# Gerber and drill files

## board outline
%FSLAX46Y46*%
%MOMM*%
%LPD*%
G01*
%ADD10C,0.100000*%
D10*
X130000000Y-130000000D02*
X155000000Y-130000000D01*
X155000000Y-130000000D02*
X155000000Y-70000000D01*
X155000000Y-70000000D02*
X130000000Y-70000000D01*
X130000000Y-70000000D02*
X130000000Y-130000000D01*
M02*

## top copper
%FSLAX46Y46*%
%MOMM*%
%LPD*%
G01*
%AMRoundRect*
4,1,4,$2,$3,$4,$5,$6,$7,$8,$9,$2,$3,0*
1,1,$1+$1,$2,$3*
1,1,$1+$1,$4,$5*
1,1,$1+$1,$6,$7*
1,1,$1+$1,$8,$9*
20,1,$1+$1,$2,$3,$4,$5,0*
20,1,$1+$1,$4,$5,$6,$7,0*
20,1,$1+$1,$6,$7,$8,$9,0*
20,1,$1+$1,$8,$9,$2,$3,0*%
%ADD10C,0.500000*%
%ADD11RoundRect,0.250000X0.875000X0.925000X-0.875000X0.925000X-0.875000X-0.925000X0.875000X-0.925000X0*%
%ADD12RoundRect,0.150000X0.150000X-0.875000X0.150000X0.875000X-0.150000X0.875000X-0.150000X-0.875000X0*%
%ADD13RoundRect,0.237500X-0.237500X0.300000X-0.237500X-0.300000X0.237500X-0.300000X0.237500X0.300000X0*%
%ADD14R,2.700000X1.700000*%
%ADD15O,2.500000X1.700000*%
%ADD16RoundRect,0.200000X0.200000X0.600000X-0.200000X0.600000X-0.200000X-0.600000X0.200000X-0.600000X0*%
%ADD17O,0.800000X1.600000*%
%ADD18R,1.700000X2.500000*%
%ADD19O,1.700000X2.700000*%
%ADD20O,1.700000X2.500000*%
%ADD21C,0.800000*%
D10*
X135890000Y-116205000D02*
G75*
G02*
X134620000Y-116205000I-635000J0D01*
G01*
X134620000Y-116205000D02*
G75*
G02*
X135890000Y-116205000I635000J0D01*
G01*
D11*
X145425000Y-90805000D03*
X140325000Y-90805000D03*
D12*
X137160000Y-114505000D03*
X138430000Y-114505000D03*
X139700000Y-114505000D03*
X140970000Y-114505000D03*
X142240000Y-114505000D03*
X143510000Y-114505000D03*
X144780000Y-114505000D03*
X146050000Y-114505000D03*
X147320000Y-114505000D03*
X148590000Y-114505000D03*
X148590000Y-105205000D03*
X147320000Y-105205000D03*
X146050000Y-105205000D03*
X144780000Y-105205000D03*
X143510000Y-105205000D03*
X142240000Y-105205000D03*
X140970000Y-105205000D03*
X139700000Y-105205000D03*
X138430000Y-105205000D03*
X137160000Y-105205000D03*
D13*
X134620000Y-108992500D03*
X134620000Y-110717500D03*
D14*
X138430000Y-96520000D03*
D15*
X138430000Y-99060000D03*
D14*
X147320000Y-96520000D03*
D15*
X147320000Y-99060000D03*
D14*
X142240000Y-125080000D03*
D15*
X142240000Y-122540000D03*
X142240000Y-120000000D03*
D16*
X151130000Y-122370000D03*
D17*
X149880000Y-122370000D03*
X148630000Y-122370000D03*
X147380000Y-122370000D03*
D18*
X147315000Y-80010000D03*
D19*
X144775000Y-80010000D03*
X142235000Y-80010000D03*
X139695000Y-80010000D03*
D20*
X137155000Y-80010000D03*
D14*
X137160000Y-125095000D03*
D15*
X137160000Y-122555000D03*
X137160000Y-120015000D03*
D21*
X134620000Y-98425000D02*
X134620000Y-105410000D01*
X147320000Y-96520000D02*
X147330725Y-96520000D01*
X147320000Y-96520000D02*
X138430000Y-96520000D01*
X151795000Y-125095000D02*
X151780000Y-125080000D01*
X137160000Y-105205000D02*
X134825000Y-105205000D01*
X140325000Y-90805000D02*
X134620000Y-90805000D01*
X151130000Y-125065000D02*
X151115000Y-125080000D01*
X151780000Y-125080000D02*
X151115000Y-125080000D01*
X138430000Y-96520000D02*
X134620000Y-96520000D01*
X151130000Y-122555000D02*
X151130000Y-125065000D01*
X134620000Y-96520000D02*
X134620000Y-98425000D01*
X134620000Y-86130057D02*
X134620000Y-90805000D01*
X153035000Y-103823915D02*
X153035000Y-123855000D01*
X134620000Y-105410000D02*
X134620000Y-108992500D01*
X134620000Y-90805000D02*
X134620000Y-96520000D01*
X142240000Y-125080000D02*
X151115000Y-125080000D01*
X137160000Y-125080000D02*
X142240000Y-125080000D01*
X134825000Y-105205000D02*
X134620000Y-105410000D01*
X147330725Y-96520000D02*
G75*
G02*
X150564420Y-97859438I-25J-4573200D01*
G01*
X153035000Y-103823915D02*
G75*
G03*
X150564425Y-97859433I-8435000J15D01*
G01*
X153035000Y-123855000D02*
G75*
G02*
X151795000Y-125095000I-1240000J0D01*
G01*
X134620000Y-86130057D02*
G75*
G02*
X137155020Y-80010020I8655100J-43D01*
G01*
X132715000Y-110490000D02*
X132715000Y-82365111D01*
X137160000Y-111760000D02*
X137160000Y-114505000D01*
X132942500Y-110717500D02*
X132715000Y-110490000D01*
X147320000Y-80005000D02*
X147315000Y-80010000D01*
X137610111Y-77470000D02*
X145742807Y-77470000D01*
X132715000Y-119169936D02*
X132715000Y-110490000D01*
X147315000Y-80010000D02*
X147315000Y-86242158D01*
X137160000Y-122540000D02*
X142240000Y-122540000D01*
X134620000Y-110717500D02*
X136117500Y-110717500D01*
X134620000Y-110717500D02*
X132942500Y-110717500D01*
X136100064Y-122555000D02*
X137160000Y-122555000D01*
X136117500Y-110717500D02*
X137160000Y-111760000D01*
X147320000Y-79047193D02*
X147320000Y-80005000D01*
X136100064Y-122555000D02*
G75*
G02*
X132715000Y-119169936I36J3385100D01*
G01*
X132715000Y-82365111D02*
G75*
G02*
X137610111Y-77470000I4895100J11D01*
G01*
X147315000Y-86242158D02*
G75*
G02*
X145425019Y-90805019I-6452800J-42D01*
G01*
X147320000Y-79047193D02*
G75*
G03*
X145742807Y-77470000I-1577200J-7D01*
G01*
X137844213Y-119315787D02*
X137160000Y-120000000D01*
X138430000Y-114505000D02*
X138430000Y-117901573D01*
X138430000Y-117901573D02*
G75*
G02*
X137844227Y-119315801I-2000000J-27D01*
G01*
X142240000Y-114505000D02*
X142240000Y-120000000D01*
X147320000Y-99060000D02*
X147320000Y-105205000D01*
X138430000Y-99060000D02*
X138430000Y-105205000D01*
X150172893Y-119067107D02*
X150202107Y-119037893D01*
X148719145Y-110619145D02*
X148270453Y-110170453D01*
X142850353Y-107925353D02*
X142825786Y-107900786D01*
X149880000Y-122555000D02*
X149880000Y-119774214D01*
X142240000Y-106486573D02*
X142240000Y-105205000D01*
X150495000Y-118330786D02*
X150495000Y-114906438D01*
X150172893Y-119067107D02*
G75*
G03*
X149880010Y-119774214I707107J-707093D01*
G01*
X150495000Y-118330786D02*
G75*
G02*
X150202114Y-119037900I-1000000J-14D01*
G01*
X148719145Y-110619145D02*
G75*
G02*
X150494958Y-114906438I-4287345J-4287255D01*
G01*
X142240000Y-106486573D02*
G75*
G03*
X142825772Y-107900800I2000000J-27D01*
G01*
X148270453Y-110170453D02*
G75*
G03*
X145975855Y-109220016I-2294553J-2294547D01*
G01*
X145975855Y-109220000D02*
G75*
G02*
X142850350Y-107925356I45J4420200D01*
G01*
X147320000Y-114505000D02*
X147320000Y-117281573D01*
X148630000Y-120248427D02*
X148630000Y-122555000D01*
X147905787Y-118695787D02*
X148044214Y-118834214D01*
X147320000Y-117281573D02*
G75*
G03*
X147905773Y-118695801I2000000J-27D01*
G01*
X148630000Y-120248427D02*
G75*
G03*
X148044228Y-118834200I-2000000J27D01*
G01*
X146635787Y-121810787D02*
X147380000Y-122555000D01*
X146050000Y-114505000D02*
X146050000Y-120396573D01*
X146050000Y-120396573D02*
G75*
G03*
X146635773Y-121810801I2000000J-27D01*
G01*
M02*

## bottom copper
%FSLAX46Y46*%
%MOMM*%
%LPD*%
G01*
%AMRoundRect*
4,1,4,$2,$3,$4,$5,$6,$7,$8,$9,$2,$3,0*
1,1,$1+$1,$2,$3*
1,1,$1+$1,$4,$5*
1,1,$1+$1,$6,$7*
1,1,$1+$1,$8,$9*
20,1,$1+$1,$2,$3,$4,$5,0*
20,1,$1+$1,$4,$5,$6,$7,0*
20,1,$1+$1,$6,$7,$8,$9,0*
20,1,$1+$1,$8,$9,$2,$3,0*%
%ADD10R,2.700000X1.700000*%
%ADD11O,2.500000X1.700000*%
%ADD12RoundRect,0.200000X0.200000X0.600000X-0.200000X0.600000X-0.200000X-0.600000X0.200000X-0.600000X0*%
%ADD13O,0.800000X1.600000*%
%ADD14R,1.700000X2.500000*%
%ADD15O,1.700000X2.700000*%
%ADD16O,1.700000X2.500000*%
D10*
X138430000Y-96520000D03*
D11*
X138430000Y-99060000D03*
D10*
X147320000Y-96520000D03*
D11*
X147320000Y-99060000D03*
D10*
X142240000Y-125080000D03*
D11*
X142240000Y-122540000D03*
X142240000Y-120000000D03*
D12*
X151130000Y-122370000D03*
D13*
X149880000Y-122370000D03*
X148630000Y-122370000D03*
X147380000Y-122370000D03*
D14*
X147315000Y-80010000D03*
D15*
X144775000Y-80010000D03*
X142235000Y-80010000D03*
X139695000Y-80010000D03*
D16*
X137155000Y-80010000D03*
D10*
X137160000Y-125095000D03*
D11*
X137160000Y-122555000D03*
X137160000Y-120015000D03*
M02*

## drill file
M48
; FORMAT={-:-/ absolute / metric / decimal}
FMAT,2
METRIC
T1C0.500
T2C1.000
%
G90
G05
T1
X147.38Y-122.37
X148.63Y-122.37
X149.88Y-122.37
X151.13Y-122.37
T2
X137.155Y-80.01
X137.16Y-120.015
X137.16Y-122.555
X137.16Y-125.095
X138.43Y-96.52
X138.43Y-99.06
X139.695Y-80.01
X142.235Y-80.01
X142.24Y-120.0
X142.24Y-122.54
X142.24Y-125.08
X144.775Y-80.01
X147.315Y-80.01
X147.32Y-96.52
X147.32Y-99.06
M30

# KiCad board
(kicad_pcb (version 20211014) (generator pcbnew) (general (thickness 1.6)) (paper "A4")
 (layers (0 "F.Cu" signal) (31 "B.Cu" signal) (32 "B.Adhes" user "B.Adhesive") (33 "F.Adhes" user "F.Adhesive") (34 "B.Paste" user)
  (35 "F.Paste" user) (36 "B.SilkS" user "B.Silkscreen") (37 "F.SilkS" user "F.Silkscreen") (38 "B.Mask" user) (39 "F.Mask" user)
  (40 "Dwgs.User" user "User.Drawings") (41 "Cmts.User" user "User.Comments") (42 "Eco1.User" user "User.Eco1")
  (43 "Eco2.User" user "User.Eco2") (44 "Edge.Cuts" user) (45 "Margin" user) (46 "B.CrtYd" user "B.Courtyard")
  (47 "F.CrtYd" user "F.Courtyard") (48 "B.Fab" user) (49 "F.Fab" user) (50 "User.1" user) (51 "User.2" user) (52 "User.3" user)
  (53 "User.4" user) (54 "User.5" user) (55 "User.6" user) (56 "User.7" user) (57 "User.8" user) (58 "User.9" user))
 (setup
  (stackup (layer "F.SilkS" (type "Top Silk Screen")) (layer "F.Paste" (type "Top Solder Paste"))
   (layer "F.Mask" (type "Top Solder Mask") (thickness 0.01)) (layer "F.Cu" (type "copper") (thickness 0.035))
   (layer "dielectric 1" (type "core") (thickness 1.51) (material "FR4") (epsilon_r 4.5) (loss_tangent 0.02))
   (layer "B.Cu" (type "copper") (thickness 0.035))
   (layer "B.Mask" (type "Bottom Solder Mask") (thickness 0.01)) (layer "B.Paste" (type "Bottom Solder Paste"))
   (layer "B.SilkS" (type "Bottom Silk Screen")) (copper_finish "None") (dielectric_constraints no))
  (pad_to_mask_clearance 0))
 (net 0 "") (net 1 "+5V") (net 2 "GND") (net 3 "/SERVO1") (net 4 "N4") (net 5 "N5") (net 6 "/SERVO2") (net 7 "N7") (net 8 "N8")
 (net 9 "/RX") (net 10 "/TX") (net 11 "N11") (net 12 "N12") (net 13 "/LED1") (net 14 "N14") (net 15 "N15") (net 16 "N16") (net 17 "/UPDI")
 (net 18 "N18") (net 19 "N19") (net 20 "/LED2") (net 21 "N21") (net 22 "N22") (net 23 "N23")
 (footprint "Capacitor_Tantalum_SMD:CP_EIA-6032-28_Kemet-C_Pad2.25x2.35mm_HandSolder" (layer "F.Cu") (at 142.875 90.805 180)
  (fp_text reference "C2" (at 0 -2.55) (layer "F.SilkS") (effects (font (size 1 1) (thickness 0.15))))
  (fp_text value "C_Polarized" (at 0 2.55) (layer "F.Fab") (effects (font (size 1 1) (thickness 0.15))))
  (pad "1" smd roundrect locked (at -2.55 0 180) (size 2.25 2.35) (layers "F.Cu" "F.Paste" "F.Mask") (roundrect_rratio 0.111111)
   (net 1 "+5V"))
  (pad "2" smd roundrect locked (at 2.55 0 180) (size 2.25 2.35) (layers "F.Cu" "F.Paste" "F.Mask") (roundrect_rratio 0.111111)
   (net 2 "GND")))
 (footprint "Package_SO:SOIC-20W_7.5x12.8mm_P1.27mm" (layer "F.Cu") (at 142.875 109.855 90)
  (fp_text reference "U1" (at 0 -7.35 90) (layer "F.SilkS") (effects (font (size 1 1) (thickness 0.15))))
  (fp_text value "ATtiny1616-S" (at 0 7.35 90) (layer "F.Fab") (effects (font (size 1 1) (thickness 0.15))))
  (pad "1" smd roundrect locked (at -4.65 -5.715 90) (size 2.05 0.6) (layers "F.Cu" "F.Paste" "F.Mask") (roundrect_rratio 0.25)
   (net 1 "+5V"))
  (pad "2" smd roundrect locked (at -4.65 -4.445 90) (size 2.05 0.6) (layers "F.Cu" "F.Paste" "F.Mask") (roundrect_rratio 0.25)
   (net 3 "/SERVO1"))
  (pad "3" smd roundrect locked (at -4.65 -3.175 90) (size 2.05 0.6) (layers "F.Cu" "F.Paste" "F.Mask") (roundrect_rratio 0.25) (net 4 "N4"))
  (pad "4" smd roundrect locked (at -4.65 -1.905 90) (size 2.05 0.6) (layers "F.Cu" "F.Paste" "F.Mask") (roundrect_rratio 0.25) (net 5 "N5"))
  (pad "5" smd roundrect locked (at -4.65 -0.635 90) (size 2.05 0.6) (layers "F.Cu" "F.Paste" "F.Mask") (roundrect_rratio 0.25)
   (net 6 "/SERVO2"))
  (pad "6" smd roundrect locked (at -4.65 0.635 90) (size 2.05 0.6) (layers "F.Cu" "F.Paste" "F.Mask") (roundrect_rratio 0.25) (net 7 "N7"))
  (pad "7" smd roundrect locked (at -4.65 1.905 90) (size 2.05 0.6) (layers "F.Cu" "F.Paste" "F.Mask") (roundrect_rratio 0.25) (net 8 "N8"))
  (pad "8" smd roundrect locked (at -4.65 3.175 90) (size 2.05 0.6) (layers "F.Cu" "F.Paste" "F.Mask") (roundrect_rratio 0.25) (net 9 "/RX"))
  (pad "9" smd roundrect locked (at -4.65 4.445 90) (size 2.05 0.6) (layers "F.Cu" "F.Paste" "F.Mask") (roundrect_rratio 0.25)
   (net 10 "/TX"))
  (pad "10" smd roundrect locked (at -4.65 5.715 90) (size 2.05 0.6) (layers "F.Cu" "F.Paste" "F.Mask") (roundrect_rratio 0.25)
   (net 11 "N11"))
  (pad "11" smd roundrect locked (at 4.65 5.715 90) (size 2.05 0.6) (layers "F.Cu" "F.Paste" "F.Mask") (roundrect_rratio 0.25)
   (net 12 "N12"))
  (pad "12" smd roundrect locked (at 4.65 4.445 90) (size 2.05 0.6) (layers "F.Cu" "F.Paste" "F.Mask") (roundrect_rratio 0.25)
   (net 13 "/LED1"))
  (pad "13" smd roundrect locked (at 4.65 3.175 90) (size 2.05 0.6) (layers "F.Cu" "F.Paste" "F.Mask") (roundrect_rratio 0.25)
   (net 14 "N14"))
  (pad "14" smd roundrect locked (at 4.65 1.905 90) (size 2.05 0.6) (layers "F.Cu" "F.Paste" "F.Mask") (roundrect_rratio 0.25)
   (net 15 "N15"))
  (pad "15" smd roundrect locked (at 4.65 0.635 90) (size 2.05 0.6) (layers "F.Cu" "F.Paste" "F.Mask") (roundrect_rratio 0.25)
   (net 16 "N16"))
  (pad "16" smd roundrect locked (at 4.65 -0.635 90) (size 2.05 0.6) (layers "F.Cu" "F.Paste" "F.Mask") (roundrect_rratio 0.25)
   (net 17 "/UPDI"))
  (pad "17" smd roundrect locked (at 4.65 -1.905 90) (size 2.05 0.6) (layers "F.Cu" "F.Paste" "F.Mask") (roundrect_rratio 0.25)
   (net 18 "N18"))
  (pad "18" smd roundrect locked (at 4.65 -3.175 90) (size 2.05 0.6) (layers "F.Cu" "F.Paste" "F.Mask") (roundrect_rratio 0.25)
   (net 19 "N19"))
  (pad "19" smd roundrect locked (at 4.65 -4.445 90) (size 2.05 0.6) (layers "F.Cu" "F.Paste" "F.Mask") (roundrect_rratio 0.25)
   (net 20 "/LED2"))
  (pad "20" smd roundrect locked (at 4.65 -5.715 90) (size 2.05 0.6) (layers "F.Cu" "F.Paste" "F.Mask") (roundrect_rratio 0.25)
   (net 2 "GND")))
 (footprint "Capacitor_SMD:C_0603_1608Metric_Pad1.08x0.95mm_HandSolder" (layer "F.Cu") (at 134.62 109.855 -90)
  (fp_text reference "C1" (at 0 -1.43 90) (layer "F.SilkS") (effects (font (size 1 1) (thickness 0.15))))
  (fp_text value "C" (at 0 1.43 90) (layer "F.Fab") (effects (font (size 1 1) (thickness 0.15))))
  (pad "1" smd roundrect locked (at -0.8625 0 270) (size 1.075 0.95) (layers "F.Cu" "F.Paste" "F.Mask") (roundrect_rratio 0.25)
   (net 2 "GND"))
  (pad "2" smd roundrect locked (at 0.8625 0 270) (size 1.075 0.95) (layers "F.Cu" "F.Paste" "F.Mask") (roundrect_rratio 0.25) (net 1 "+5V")))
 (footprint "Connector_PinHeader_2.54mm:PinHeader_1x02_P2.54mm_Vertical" (layer "B.Cu") (at 138.43 96.52 180)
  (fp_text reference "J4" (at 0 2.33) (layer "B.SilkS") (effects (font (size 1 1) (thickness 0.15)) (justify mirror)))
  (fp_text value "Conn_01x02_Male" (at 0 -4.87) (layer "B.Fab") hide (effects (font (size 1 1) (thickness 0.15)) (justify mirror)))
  (pad "1" thru_hole rect locked (at 0 0 180) (size 2.7 1.7) (drill 1) (layers *.Cu *.Mask) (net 2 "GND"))
  (pad "2" thru_hole oval locked (at 0 -2.54 180) (size 2.5 1.7) (drill 1) (layers *.Cu *.Mask) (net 20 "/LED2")))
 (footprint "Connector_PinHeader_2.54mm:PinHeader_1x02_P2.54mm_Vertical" (layer "B.Cu") (at 147.32 96.52 180)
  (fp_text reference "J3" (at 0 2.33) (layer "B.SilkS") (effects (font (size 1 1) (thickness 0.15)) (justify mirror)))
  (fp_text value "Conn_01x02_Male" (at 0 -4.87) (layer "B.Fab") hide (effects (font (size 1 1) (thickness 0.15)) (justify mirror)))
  (pad "1" thru_hole rect locked (at 0 0 180) (size 2.7 1.7) (drill 1) (layers *.Cu *.Mask) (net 2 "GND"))
  (pad "2" thru_hole oval locked (at 0 -2.54 180) (size 2.5 1.7) (drill 1) (layers *.Cu *.Mask) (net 13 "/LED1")))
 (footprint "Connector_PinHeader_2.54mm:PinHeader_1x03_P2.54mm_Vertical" (layer "B.Cu") (at 142.24 125.08)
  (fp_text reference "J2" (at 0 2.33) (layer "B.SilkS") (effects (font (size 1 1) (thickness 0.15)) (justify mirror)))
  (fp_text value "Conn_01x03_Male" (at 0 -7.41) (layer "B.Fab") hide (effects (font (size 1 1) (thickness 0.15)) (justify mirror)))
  (pad "1" thru_hole rect locked (at 0 0) (size 2.7 1.7) (drill 1) (layers *.Cu *.Mask) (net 2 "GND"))
  (pad "2" thru_hole oval locked (at 0 -2.54) (size 2.5 1.7) (drill 1) (layers *.Cu *.Mask) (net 1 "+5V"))
  (pad "3" thru_hole oval locked (at 0 -5.08) (size 2.5 1.7) (drill 1) (layers *.Cu *.Mask) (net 6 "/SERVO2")))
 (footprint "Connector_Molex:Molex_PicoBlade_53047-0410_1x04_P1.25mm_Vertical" (layer "B.Cu") (at 151.13 122.37 180)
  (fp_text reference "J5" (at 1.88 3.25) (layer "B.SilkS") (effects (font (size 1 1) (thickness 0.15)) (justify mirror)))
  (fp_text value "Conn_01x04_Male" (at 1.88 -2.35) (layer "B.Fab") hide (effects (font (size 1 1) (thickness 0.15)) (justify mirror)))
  (pad "1" thru_hole roundrect locked (at 0 0 180) (size 0.8 1.6) (drill 0.5) (layers *.Cu *.Mask) (roundrect_rratio 0.25) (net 2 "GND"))
  (pad "2" thru_hole oval locked (at 1.25 0 180) (size 0.8 1.6) (drill 0.5) (layers *.Cu *.Mask) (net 17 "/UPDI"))
  (pad "3" thru_hole oval locked (at 2.5 0 180) (size 0.8 1.6) (drill 0.5) (layers *.Cu *.Mask) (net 10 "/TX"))
  (pad "4" thru_hole oval locked (at 3.75 0 180) (size 0.8 1.6) (drill 0.5) (layers *.Cu *.Mask) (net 9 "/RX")))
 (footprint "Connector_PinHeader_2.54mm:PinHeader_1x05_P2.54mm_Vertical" (layer "B.Cu") (at 147.315 80.01 90)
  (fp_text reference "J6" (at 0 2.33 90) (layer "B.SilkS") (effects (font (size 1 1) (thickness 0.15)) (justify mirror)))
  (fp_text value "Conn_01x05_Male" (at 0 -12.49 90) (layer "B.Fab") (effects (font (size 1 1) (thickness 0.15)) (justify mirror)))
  (pad "1" thru_hole rect locked (at 0 0 90) (size 2.5 1.7) (drill 1) (layers *.Cu *.Mask) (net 1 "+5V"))
  (pad "2" thru_hole oval locked (at 0 -2.54 90) (size 2.7 1.7) (drill 1) (layers *.Cu *.Mask) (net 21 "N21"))
  (pad "3" thru_hole oval locked (at 0 -5.08 90) (size 2.7 1.7) (drill 1) (layers *.Cu *.Mask) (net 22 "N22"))
  (pad "4" thru_hole oval locked (at 0 -7.62 90) (size 2.7 1.7) (drill 1) (layers *.Cu *.Mask) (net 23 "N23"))
  (pad "5" thru_hole oval locked (at 0 -10.16 90) (size 2.5 1.7) (drill 1) (layers *.Cu *.Mask) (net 2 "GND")))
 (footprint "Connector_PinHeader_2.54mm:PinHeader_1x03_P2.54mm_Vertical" (layer "B.Cu") (at 137.16 125.095)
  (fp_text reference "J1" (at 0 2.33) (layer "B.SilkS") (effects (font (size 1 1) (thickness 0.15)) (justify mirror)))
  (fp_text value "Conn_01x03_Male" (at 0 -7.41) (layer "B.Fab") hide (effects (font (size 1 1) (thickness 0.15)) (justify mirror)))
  (pad "1" thru_hole rect locked (at 0 0) (size 2.7 1.7) (drill 1) (layers *.Cu *.Mask) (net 2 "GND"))
  (pad "2" thru_hole oval locked (at 0 -2.54) (size 2.5 1.7) (drill 1) (layers *.Cu *.Mask) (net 1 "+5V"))
  (pad "3" thru_hole oval locked (at 0 -5.08) (size 2.5 1.7) (drill 1) (layers *.Cu *.Mask) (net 3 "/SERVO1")))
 (gr_circle (center 135.255 116.205) (end 135.89 116.205) (layer "F.Cu") (width 0.5) (fill none))
 (gr_line (start 130 130) (end 155 130) (layer "Edge.Cuts") (width 0.1))
 (gr_line (start 155 130) (end 155 70) (layer "Edge.Cuts") (width 0.1))
 (gr_line (start 155 70) (end 130 70) (layer "Edge.Cuts") (width 0.1))
 (gr_line (start 130 70) (end 130 130) (layer "Edge.Cuts") (width 0.1))
 (segment (start 134.62 98.425) (end 134.62 105.41) (width 0.8) (layer "F.Cu") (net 2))
 (segment (start 147.32 96.52) (end 147.330725 96.52) (width 0.8) (layer "F.Cu") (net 2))
 (segment (start 147.32 96.52) (end 138.43 96.52) (width 0.8) (layer "F.Cu") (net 2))
 (segment (start 151.795 125.095) (end 151.78 125.08) (width 0.8) (layer "F.Cu") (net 2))
 (segment (start 137.16 105.205) (end 134.825 105.205) (width 0.8) (layer "F.Cu") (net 2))
 (segment (start 140.325 90.805) (end 134.62 90.805) (width 0.8) (layer "F.Cu") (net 2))
 (segment (start 151.13 125.065) (end 151.115 125.08) (width 0.8) (layer "F.Cu") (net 2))
 (segment (start 151.78 125.08) (end 151.115 125.08) (width 0.8) (layer "F.Cu") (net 2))
 (segment (start 138.43 96.52) (end 134.62 96.52) (width 0.8) (layer "F.Cu") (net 2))
 (segment (start 151.13 122.555) (end 151.13 125.065) (width 0.8) (layer "F.Cu") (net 2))
 (segment (start 134.62 96.52) (end 134.62 98.425) (width 0.8) (layer "F.Cu") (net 2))
 (segment (start 134.62 86.130057) (end 134.62 90.805) (width 0.8) (layer "F.Cu") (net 2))
 (segment (start 153.035 103.823915) (end 153.035 123.855) (width 0.8) (layer "F.Cu") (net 2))
 (segment (start 134.62 105.41) (end 134.62 108.9925) (width 0.8) (layer "F.Cu") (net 2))
 (segment (start 134.62 90.805) (end 134.62 96.52) (width 0.8) (layer "F.Cu") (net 2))
 (segment (start 142.24 125.08) (end 151.115 125.08) (width 0.8) (layer "F.Cu") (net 2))
 (segment (start 137.16 125.08) (end 142.24 125.08) (width 0.8) (layer "F.Cu") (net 2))
 (segment (start 134.825 105.205) (end 134.62 105.41) (width 0.8) (layer "F.Cu") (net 2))
 (arc (start 147.330725 96.52) (mid 149.080809 96.868113) (end 150.564429 97.859429) (width 0.8) (layer "F.Cu") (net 2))
 (arc (start 153.035 103.823915) (mid 152.39292 100.595958) (end 150.564429 97.859429) (width 0.8) (layer "F.Cu") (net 2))
 (arc (start 153.035 123.855) (mid 152.671812 124.731812) (end 151.795 125.095) (width 0.8) (layer "F.Cu") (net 2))
 (arc (start 134.62 86.130057) (mid 135.27883 82.817896) (end 137.155 80.01) (width 0.8) (layer "F.Cu") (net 2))
 (segment (start 132.715 110.49) (end 132.715 82.365111) (width 0.8) (layer "F.Cu") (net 1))
 (segment (start 137.16 111.76) (end 137.16 114.505) (width 0.8) (layer "F.Cu") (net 1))
 (segment (start 132.9425 110.7175) (end 132.715 110.49) (width 0.8) (layer "F.Cu") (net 1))
 (segment (start 147.32 80.005) (end 147.315 80.01) (width 0.8) (layer "F.Cu") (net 1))
 (segment (start 137.610111 77.47) (end 145.742807 77.47) (width 0.8) (layer "F.Cu") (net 1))
 (segment (start 132.715 119.169936) (end 132.715 110.49) (width 0.8) (layer "F.Cu") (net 1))
 (segment (start 147.315 80.01) (end 147.315 86.242158) (width 0.8) (layer "F.Cu") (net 1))
 (segment (start 137.16 122.54) (end 142.24 122.54) (width 0.8) (layer "F.Cu") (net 1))
 (segment (start 134.62 110.7175) (end 136.1175 110.7175) (width 0.8) (layer "F.Cu") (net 1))
 (segment (start 134.62 110.7175) (end 132.9425 110.7175) (width 0.8) (layer "F.Cu") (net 1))
 (segment (start 136.100064 122.555) (end 137.16 122.555) (width 0.8) (layer "F.Cu") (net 1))
 (segment (start 136.1175 110.7175) (end 137.16 111.76) (width 0.8) (layer "F.Cu") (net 1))
 (segment (start 147.32 79.047193) (end 147.32 80.005) (width 0.8) (layer "F.Cu") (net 1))
 (arc (start 136.100064 122.555) (mid 133.706462 121.563538) (end 132.715 119.169936) (width 0.8) (layer "F.Cu") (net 1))
 (arc (start 132.715 82.365111) (mid 134.148745 78.903745) (end 137.610111 77.47) (width 0.8) (layer "F.Cu") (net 1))
 (arc (start 147.315 86.242158) (mid 146.823809 88.711541) (end 145.425 90.805) (width 0.8) (layer "F.Cu") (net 1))
 (arc (start 147.32 79.047193) (mid 146.858051 77.931949) (end 145.742807 77.47) (width 0.8) (layer "F.Cu") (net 1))
 (segment (start 137.844213 119.315787) (end 137.16 120) (width 0.8) (layer "F.Cu") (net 3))
 (segment (start 138.43 114.505) (end 138.43 117.901573) (width 0.8) (layer "F.Cu") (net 3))
 (arc (start 138.43 117.901573) (mid 138.277759 118.66694) (end 137.844213 119.315787) (width 0.8) (layer "F.Cu") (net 3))
 (segment (start 142.24 114.505) (end 142.24 120) (width 0.8) (layer "F.Cu") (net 6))
 (segment (start 147.32 99.06) (end 147.32 105.205) (width 0.8) (layer "F.Cu") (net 13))
 (segment (start 138.43 99.06) (end 138.43 105.205) (width 0.8) (layer "F.Cu") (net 20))
 (segment (start 150.172893 119.067107) (end 150.202107 119.037893) (width 0.8) (layer "F.Cu") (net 17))
 (segment (start 148.719145 110.619145) (end 148.270453 110.170453) (width 0.8) (layer "F.Cu") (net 17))
 (segment (start 142.850353 107.925353) (end 142.825786 107.900786) (width 0.8) (layer "F.Cu") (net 17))
 (segment (start 149.88 122.555) (end 149.88 119.774214) (width 0.8) (layer "F.Cu") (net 17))
 (segment (start 142.24 106.486573) (end 142.24 105.205) (width 0.8) (layer "F.Cu") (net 17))
 (segment (start 150.495 118.330786) (end 150.495 114.906438) (width 0.8) (layer "F.Cu") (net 17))
 (arc (start 150.172893 119.067107) (mid 149.95612 119.39153) (end 149.88 119.774214) (width 0.8) (layer "F.Cu") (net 17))
 (arc (start 150.495 118.330786) (mid 150.41888 118.713469) (end 150.202107 119.037893) (width 0.8) (layer "F.Cu") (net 17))
 (arc (start 148.719145 110.619145) (mid 150.03347 112.586172) (end 150.495 114.906438) (width 0.8) (layer "F.Cu") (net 17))
 (arc (start 142.24 106.486573) (mid 142.392241 107.25194) (end 142.825786 107.900786) (width 0.8) (layer "F.Cu") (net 17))
 (arc (start 148.270453 110.170453) (mid 147.217682 109.467014) (end 145.975855 109.22) (width 0.8) (layer "F.Cu") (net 17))
 (arc (start 145.975855 109.22) (mid 144.284368 108.883532) (end 142.850353 107.925353) (width 0.8) (layer "F.Cu") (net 17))
 (segment (start 147.32 114.505) (end 147.32 117.281573) (width 0.8) (layer "F.Cu") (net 10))
 (segment (start 148.63 120.248427) (end 148.63 122.555) (width 0.8) (layer "F.Cu") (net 10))
 (segment (start 147.905787 118.695787) (end 148.044214 118.834214) (width 0.8) (layer "F.Cu") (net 10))
 (arc (start 147.32 117.281573) (mid 147.472241 118.04694) (end 147.905787 118.695787) (width 0.8) (layer "F.Cu") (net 10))
 (arc (start 148.63 120.248427) (mid 148.477759 119.48306) (end 148.044214 118.834214) (width 0.8) (layer "F.Cu") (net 10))
 (segment (start 146.635787 121.810787) (end 147.38 122.555) (width 0.8) (layer "F.Cu") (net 9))
 (segment (start 146.05 114.505) (end 146.05 120.396573) (width 0.8) (layer "F.Cu") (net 9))
 (arc (start 146.05 120.396573) (mid 146.202241 121.16194) (end 146.635787 121.810787) (width 0.8) (layer "F.Cu") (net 9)))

